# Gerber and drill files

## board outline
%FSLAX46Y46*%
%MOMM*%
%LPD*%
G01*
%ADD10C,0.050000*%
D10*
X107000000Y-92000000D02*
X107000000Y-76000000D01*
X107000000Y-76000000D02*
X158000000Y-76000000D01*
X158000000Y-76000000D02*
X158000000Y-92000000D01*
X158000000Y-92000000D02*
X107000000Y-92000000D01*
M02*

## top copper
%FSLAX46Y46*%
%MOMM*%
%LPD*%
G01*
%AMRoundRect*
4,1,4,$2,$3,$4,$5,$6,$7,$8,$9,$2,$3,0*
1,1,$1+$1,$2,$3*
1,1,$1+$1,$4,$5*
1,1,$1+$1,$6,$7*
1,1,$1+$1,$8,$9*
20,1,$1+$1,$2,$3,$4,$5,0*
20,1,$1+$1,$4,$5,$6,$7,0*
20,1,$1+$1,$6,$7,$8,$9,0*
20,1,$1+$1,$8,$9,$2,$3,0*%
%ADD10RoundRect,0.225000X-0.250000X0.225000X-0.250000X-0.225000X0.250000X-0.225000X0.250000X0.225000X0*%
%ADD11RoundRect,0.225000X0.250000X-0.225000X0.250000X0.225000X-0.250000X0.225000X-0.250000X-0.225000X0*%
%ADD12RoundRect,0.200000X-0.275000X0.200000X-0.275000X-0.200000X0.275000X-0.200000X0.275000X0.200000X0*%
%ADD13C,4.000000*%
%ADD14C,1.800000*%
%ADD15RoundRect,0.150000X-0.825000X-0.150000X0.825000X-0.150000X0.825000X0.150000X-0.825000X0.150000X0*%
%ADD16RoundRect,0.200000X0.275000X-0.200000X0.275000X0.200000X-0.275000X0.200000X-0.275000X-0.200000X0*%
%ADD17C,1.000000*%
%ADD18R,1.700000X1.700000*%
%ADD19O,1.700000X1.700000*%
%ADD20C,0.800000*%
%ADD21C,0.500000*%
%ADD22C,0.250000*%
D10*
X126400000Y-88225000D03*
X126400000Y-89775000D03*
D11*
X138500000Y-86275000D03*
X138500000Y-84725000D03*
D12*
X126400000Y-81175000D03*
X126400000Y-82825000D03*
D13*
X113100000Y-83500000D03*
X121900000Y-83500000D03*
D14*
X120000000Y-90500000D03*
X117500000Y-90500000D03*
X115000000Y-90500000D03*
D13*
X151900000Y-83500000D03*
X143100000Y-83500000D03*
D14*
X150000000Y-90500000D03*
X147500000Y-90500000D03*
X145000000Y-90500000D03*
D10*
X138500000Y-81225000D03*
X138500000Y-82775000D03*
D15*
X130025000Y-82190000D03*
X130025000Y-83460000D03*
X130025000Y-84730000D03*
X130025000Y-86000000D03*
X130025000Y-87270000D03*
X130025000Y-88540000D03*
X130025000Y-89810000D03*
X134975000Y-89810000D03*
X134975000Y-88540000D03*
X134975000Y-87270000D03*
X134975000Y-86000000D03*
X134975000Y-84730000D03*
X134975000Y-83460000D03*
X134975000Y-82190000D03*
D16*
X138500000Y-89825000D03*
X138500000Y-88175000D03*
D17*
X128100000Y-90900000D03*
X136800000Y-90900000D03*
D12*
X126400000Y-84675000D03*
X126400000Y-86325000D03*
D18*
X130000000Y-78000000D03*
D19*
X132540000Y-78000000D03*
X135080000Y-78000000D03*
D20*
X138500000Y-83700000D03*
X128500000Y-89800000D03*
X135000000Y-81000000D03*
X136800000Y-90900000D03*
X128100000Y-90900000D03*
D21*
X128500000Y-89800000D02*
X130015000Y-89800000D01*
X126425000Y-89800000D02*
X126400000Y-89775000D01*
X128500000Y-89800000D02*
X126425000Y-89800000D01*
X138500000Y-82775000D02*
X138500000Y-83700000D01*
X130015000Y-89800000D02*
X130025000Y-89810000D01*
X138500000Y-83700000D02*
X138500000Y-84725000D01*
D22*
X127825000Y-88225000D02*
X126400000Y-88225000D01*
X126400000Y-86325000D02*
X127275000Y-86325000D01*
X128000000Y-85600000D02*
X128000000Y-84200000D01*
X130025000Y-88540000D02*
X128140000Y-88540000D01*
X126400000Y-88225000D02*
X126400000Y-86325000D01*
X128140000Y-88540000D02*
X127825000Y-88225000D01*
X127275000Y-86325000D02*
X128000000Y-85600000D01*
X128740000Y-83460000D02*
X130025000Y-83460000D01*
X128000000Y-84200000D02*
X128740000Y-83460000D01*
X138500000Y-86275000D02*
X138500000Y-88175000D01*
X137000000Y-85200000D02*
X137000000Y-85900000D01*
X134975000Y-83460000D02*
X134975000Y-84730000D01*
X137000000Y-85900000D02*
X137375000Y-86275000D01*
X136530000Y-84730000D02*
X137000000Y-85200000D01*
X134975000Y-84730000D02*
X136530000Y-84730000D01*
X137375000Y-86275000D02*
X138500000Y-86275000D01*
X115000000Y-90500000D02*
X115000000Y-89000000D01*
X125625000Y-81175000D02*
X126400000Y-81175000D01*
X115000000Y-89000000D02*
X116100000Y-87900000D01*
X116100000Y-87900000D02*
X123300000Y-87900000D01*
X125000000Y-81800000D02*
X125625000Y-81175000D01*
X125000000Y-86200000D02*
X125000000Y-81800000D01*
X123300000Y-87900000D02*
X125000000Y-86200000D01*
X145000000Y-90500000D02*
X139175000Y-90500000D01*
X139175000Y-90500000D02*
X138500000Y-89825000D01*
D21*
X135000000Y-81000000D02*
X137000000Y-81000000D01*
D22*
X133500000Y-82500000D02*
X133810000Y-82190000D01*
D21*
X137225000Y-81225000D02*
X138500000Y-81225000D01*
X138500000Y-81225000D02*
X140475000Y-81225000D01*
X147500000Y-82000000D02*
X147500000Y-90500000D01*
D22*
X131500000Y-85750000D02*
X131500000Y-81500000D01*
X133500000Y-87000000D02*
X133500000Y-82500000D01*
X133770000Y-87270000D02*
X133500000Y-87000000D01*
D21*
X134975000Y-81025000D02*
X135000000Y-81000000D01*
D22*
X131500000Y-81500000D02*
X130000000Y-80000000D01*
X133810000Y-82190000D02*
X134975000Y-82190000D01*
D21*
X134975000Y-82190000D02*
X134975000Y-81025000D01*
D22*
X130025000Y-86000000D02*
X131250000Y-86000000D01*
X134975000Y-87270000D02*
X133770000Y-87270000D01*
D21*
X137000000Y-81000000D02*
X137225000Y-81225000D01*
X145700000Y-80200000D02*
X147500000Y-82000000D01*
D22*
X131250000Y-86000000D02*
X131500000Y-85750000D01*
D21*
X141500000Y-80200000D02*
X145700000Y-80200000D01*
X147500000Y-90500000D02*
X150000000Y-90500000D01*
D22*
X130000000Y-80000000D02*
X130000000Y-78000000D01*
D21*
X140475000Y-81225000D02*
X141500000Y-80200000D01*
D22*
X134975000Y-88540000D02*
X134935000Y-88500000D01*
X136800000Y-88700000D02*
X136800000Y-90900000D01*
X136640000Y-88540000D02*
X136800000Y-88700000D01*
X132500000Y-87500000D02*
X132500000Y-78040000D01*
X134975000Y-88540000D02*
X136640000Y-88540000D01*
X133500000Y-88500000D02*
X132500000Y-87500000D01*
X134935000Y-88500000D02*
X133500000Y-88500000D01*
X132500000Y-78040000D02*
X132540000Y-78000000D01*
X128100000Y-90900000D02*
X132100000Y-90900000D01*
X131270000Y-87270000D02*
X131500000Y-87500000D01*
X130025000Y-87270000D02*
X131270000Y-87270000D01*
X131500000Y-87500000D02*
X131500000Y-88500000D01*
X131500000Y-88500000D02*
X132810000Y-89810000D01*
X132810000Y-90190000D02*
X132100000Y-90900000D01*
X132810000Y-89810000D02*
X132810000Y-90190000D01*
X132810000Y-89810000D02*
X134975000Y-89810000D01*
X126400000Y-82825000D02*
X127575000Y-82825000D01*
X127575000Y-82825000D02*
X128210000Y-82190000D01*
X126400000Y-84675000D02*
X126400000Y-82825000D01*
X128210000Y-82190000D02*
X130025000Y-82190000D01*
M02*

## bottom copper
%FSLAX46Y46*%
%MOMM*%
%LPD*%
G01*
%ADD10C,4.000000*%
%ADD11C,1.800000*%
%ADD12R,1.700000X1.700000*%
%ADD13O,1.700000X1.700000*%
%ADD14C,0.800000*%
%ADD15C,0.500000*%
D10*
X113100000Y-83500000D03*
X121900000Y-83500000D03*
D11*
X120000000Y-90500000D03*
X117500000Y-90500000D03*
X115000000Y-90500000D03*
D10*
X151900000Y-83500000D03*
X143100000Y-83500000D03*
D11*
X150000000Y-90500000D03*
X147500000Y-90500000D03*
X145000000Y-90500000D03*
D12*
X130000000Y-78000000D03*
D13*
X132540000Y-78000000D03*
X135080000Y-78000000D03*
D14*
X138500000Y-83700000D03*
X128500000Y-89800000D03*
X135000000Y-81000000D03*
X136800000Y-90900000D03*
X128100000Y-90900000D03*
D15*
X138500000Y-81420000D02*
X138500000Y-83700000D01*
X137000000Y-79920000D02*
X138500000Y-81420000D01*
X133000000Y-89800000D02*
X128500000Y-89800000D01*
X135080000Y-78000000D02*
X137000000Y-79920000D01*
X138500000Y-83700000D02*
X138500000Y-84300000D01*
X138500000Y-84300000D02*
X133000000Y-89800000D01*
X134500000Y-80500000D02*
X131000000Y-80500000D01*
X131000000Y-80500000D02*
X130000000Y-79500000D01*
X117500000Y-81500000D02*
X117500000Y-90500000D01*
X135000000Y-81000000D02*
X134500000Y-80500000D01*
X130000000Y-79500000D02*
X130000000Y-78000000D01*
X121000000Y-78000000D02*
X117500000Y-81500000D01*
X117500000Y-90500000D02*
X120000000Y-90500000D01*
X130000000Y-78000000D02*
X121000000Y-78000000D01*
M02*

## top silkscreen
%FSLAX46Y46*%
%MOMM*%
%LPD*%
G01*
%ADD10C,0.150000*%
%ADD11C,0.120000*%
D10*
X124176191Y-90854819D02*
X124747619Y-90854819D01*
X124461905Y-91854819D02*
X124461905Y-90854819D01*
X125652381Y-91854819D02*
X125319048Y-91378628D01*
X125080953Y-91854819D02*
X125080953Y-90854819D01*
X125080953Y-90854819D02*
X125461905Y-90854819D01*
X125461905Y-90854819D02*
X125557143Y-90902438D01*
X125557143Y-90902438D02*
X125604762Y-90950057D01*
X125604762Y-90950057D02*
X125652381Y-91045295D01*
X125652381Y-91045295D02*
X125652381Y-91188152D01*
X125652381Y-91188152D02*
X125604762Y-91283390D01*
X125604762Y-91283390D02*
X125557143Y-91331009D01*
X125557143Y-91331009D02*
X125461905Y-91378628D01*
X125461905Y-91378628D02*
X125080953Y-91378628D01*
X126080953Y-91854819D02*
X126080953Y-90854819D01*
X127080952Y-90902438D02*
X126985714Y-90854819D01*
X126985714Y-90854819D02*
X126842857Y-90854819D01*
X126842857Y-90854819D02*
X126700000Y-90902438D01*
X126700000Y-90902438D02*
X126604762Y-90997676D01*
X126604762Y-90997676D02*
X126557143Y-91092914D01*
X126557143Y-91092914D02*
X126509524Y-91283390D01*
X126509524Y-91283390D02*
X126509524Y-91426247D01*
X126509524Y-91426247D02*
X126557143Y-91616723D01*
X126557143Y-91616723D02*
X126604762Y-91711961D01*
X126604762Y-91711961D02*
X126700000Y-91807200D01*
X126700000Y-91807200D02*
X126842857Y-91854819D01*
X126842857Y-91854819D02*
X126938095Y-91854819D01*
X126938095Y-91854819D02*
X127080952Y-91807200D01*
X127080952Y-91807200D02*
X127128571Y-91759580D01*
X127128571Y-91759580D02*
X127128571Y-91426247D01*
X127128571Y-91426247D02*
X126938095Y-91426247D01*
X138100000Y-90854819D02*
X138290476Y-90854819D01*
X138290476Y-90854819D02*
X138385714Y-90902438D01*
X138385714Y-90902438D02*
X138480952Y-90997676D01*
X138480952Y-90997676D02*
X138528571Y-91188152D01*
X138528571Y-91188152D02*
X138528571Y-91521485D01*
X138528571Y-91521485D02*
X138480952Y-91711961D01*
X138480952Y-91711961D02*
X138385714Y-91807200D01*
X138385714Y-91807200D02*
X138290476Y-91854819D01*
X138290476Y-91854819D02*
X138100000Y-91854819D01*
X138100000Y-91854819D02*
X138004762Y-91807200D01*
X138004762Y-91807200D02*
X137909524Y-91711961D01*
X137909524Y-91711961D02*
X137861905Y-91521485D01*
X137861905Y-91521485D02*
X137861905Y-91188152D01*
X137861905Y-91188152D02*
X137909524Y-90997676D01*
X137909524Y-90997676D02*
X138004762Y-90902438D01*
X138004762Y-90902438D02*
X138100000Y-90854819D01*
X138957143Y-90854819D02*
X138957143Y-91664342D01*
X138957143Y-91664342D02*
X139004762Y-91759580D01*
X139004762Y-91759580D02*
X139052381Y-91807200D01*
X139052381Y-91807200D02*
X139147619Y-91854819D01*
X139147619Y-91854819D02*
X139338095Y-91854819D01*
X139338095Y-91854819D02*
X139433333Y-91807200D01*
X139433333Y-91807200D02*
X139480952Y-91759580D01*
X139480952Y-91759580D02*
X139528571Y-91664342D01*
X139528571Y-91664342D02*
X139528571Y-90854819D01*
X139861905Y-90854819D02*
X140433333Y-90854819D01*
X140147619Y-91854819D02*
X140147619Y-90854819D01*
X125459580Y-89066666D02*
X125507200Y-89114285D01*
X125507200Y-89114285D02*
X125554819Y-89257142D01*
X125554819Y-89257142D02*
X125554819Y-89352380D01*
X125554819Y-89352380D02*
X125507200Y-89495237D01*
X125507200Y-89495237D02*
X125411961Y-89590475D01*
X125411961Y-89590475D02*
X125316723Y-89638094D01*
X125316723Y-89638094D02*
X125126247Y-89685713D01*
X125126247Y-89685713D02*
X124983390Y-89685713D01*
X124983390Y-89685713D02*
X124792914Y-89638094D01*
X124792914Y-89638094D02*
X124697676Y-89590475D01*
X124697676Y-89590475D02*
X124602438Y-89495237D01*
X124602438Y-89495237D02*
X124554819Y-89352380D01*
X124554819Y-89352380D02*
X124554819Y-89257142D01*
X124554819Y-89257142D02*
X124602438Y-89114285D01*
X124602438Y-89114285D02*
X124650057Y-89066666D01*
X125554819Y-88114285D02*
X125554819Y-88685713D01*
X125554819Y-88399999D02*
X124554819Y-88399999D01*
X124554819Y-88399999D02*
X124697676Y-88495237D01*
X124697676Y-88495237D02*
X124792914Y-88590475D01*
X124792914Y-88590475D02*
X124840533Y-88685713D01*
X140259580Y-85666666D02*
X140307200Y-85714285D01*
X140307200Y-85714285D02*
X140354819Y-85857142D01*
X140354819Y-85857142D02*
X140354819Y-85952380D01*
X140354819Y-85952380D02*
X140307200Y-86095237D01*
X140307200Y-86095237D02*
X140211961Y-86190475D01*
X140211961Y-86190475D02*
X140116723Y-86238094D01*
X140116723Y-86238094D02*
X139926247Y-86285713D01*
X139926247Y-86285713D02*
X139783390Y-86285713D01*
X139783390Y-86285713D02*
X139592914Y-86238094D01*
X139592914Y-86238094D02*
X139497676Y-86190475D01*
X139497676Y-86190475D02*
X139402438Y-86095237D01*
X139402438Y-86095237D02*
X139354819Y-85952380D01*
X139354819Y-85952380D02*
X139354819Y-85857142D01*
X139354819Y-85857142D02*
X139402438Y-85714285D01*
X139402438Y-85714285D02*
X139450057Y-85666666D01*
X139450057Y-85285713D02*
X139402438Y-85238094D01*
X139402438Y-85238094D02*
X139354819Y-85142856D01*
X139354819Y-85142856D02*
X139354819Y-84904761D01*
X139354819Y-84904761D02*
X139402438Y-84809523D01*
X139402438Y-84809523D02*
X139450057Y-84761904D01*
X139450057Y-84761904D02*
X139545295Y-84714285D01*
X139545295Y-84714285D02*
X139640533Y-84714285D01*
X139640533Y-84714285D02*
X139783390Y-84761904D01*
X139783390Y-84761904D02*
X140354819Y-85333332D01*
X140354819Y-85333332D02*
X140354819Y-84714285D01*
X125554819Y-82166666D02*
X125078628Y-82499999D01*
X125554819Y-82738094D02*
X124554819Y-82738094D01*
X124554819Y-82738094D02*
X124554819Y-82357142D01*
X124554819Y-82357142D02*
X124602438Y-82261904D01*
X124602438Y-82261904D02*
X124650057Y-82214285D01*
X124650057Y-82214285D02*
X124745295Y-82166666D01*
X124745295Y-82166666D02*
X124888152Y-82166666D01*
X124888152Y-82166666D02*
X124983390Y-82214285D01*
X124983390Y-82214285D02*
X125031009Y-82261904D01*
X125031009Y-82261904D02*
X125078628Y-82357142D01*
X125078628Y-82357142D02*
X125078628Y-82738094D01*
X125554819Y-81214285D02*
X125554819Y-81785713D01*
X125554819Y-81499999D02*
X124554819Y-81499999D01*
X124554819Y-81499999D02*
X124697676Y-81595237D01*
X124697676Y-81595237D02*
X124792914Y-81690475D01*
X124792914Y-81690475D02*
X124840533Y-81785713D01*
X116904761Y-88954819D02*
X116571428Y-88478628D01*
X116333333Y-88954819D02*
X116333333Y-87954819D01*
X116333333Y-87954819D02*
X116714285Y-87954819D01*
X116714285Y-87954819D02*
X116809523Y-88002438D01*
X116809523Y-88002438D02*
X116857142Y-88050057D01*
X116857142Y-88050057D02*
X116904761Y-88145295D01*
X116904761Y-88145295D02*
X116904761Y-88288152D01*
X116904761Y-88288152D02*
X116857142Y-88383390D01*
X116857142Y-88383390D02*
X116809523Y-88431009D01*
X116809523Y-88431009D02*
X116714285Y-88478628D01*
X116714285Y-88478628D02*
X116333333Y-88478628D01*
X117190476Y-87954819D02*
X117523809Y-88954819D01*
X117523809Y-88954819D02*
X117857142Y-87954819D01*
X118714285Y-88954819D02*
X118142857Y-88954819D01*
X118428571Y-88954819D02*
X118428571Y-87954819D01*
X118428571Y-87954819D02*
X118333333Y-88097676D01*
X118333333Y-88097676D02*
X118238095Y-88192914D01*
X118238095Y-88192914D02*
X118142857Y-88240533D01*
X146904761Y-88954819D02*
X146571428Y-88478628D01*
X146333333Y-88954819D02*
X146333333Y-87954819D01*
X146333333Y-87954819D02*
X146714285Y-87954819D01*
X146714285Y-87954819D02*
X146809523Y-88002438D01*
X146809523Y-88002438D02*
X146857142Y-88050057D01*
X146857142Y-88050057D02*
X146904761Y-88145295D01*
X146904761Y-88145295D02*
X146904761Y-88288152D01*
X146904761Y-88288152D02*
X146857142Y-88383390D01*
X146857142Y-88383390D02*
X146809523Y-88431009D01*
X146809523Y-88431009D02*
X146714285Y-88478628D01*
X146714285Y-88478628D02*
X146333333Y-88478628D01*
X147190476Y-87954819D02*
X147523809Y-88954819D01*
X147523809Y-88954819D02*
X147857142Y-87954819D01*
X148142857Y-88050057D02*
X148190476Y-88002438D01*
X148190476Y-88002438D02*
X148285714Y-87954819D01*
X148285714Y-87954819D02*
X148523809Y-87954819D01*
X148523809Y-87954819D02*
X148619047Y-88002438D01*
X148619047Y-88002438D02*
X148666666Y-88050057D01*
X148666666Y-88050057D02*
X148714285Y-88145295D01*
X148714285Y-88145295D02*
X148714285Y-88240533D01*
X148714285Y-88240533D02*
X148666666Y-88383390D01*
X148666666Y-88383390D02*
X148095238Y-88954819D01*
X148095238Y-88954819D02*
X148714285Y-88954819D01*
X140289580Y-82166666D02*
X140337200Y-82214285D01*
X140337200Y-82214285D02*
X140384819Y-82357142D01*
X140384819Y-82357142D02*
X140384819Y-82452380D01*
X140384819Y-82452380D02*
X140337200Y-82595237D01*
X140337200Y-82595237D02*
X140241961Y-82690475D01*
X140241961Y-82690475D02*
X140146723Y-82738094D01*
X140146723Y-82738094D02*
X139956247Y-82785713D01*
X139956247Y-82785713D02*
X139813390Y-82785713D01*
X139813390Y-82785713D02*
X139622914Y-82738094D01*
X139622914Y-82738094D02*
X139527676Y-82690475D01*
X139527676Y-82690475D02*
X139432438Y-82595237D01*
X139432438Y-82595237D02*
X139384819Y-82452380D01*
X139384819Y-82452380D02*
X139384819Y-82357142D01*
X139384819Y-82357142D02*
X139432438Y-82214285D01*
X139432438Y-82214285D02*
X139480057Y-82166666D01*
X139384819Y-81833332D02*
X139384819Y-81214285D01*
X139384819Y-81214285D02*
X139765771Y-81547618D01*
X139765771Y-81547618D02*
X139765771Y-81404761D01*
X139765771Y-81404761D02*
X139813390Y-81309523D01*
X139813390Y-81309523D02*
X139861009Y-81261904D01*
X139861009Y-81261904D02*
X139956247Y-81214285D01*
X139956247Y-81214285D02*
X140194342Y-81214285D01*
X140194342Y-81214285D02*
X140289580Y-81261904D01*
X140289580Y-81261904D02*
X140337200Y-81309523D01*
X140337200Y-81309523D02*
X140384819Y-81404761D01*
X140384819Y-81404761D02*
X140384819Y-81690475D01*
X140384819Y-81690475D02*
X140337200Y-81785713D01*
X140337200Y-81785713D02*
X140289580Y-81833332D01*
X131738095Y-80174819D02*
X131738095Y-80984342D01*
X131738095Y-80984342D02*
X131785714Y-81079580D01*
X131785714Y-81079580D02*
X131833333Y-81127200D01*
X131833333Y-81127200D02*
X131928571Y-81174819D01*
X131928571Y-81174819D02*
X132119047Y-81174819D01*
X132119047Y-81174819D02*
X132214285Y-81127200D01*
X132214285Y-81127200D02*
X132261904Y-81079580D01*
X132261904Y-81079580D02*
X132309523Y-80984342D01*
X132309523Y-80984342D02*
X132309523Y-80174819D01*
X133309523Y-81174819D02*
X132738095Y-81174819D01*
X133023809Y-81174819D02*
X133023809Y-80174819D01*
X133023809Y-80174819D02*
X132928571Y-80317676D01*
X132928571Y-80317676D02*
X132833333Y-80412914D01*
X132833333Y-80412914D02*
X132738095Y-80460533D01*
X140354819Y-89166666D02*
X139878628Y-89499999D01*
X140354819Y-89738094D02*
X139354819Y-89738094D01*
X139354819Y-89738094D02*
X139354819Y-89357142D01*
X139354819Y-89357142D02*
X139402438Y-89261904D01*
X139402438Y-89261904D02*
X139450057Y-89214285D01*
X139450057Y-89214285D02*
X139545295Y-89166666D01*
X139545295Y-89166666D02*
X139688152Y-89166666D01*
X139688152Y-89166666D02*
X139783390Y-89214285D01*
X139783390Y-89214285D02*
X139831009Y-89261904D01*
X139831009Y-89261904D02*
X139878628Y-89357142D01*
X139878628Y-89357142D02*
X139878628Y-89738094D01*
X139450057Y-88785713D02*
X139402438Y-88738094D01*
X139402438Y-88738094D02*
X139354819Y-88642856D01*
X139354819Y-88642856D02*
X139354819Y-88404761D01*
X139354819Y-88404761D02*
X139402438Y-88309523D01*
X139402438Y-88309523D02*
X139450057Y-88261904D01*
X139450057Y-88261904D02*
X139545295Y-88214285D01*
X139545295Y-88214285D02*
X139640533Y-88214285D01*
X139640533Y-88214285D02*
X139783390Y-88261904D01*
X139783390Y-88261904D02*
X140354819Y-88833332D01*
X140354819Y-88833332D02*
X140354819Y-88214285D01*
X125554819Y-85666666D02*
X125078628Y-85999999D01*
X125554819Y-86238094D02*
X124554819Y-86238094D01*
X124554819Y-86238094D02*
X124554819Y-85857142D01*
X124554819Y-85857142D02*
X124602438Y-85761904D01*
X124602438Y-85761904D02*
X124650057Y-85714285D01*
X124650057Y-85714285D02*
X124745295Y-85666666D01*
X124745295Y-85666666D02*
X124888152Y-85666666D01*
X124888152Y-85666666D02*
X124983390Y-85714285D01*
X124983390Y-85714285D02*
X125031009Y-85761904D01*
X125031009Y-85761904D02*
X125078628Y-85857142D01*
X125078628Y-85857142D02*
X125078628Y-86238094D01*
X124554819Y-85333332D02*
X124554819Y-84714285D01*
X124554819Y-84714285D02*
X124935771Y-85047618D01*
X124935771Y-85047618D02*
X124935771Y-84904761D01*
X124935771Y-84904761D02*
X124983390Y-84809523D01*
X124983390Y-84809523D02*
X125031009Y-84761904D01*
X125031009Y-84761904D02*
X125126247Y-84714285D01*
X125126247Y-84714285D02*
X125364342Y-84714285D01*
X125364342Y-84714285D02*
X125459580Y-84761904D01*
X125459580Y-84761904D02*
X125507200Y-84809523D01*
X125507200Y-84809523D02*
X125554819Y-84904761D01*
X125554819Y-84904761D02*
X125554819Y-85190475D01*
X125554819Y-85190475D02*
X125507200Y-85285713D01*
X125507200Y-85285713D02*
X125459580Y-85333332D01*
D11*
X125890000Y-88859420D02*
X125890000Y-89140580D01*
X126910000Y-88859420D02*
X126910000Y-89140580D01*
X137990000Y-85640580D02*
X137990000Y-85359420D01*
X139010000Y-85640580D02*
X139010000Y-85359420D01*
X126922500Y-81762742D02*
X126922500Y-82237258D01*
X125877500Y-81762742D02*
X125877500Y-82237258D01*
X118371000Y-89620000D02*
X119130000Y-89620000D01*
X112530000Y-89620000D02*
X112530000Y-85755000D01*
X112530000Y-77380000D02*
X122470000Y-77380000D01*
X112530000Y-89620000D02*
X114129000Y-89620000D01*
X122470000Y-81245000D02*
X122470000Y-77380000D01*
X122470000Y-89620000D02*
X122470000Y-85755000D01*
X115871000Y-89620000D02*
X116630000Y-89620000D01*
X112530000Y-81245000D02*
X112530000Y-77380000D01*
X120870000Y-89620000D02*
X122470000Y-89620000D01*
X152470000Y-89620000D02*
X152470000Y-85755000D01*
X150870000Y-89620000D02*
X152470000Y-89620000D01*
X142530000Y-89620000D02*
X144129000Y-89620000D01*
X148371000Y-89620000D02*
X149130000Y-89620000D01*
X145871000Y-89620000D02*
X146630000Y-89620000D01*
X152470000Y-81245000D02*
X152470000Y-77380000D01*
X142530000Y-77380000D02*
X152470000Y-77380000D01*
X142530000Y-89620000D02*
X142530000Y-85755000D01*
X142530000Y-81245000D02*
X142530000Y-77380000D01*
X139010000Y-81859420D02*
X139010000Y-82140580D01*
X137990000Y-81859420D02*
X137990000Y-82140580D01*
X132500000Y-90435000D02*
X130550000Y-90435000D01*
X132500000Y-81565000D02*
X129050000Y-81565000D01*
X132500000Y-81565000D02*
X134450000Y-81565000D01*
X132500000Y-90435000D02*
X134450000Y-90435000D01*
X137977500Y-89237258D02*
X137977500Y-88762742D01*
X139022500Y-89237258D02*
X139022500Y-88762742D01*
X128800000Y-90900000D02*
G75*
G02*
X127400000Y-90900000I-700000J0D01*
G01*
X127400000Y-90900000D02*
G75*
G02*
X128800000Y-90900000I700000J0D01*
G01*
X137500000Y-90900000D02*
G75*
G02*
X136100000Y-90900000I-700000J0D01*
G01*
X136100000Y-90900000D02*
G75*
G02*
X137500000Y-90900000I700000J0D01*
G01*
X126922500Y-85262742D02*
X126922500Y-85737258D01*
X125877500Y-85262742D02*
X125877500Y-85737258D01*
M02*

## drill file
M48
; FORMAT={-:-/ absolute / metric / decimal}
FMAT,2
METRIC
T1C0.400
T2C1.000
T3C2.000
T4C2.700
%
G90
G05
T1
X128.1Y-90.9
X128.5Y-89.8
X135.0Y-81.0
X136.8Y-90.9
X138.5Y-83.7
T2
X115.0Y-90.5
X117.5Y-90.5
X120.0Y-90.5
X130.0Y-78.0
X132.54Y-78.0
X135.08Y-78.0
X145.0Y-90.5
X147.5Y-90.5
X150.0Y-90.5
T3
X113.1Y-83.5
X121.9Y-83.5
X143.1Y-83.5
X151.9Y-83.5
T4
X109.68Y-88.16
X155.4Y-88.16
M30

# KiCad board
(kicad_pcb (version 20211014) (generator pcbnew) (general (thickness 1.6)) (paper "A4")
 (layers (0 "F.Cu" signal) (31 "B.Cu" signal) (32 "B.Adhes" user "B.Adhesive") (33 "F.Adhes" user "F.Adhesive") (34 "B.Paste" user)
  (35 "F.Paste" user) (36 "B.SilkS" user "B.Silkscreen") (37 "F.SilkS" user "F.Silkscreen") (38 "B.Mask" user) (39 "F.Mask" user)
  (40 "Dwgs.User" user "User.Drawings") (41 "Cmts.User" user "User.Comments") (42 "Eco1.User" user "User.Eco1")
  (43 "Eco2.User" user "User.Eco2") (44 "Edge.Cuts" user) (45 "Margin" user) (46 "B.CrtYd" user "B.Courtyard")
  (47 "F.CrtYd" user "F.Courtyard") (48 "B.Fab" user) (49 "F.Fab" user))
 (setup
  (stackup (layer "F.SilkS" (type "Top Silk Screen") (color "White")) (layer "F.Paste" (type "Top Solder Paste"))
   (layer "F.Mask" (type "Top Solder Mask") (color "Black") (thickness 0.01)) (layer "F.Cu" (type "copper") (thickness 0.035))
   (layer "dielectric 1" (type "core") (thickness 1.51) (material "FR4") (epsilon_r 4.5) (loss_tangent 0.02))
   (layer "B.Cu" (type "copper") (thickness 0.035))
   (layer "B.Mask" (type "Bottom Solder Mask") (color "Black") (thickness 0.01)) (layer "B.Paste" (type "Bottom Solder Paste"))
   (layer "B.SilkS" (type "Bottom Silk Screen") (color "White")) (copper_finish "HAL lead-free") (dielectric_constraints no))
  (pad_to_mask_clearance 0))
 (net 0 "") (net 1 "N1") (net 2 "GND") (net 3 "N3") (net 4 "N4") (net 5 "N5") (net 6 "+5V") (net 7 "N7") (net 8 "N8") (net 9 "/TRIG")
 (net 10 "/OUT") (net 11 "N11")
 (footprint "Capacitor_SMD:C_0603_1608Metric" (layer "F.Cu") (at 126.4 89 -90)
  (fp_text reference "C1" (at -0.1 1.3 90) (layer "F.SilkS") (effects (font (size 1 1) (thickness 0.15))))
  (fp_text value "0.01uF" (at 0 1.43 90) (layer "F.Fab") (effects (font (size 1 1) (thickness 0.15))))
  (fp_line (start -0.14058 0.51) (end 0.14058 0.51) (layer "F.SilkS") (width 0.12))
  (fp_line (start -0.14058 -0.51) (end 0.14058 -0.51) (layer "F.SilkS") (width 0.12))
  (pad "1" smd roundrect locked (at -0.775 0 270) (size 0.9 0.95) (layers "F.Cu" "F.Paste" "F.Mask") (roundrect_rratio 0.25) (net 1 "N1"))
  (pad "2" smd roundrect locked (at 0.775 0 270) (size 0.9 0.95) (layers "F.Cu" "F.Paste" "F.Mask") (roundrect_rratio 0.25) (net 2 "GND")))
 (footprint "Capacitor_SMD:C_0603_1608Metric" (layer "F.Cu") (at 138.5 85.5 90)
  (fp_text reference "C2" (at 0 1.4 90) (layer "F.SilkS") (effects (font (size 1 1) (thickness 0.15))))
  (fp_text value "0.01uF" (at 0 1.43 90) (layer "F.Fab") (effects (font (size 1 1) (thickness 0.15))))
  (fp_line (start -0.14058 -0.51) (end 0.14058 -0.51) (layer "F.SilkS") (width 0.12))
  (fp_line (start -0.14058 0.51) (end 0.14058 0.51) (layer "F.SilkS") (width 0.12))
  (pad "1" smd roundrect locked (at -0.775 0 90) (size 0.9 0.95) (layers "F.Cu" "F.Paste" "F.Mask") (roundrect_rratio 0.25) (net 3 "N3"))
  (pad "2" smd roundrect locked (at 0.775 0 90) (size 0.9 0.95) (layers "F.Cu" "F.Paste" "F.Mask") (roundrect_rratio 0.25) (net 2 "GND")))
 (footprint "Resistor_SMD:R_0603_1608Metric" (layer "F.Cu") (at 126.4 82 -90)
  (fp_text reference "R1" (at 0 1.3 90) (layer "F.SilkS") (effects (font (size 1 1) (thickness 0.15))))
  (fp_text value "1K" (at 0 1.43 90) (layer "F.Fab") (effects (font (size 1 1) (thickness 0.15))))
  (fp_line (start -0.237258 -0.5225) (end 0.237258 -0.5225) (layer "F.SilkS") (width 0.12))
  (fp_line (start -0.237258 0.5225) (end 0.237258 0.5225) (layer "F.SilkS") (width 0.12))
  (pad "1" smd roundrect locked (at -0.825 0 270) (size 0.8 0.95) (layers "F.Cu" "F.Paste" "F.Mask") (roundrect_rratio 0.25) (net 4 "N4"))
  (pad "2" smd roundrect locked (at 0.825 0 270) (size 0.8 0.95) (layers "F.Cu" "F.Paste" "F.Mask") (roundrect_rratio 0.25) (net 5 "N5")))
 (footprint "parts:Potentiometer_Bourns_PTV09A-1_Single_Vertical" (layer "F.Cu") (at 120 90.5 90)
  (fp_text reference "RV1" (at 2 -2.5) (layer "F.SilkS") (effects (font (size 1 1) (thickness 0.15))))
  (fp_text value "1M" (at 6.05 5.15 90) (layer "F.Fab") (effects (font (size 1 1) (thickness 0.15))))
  (fp_line (start 0.88 -1.629) (end 0.88 -0.87) (layer "F.SilkS") (width 0.12))
  (fp_line (start 0.88 -7.47) (end 4.745 -7.47) (layer "F.SilkS") (width 0.12))
  (fp_line (start 13.12 -7.47) (end 13.12 2.47) (layer "F.SilkS") (width 0.12))
  (fp_line (start 0.88 -7.47) (end 0.88 -5.871) (layer "F.SilkS") (width 0.12))
  (fp_line (start 9.255 2.47) (end 13.12 2.47) (layer "F.SilkS") (width 0.12))
  (fp_line (start 0.88 2.47) (end 4.745 2.47) (layer "F.SilkS") (width 0.12))
  (fp_line (start 0.88 -4.129) (end 0.88 -3.37) (layer "F.SilkS") (width 0.12))
  (fp_line (start 9.255 -7.47) (end 13.12 -7.47) (layer "F.SilkS") (width 0.12))
  (fp_line (start 0.88 0.87) (end 0.88 2.47) (layer "F.SilkS") (width 0.12))
  (pad "" np_thru_hole circle locked (at 7 -6.9 90) (size 4 4) (drill 2) (layers *.Cu *.Mask))
  (pad "" np_thru_hole circle locked (at 7 1.9 90) (size 4 4) (drill 2) (layers *.Cu *.Mask))
  (pad "1" thru_hole circle locked (at 0 0 90) (size 1.8 1.8) (drill 1) (layers *.Cu *.Mask) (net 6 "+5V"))
  (pad "2" thru_hole circle locked (at 0 -2.5 90) (size 1.8 1.8) (drill 1) (layers *.Cu *.Mask) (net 6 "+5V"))
  (pad "3" thru_hole circle locked (at 0 -5 90) (size 1.8 1.8) (drill 1) (layers *.Cu *.Mask) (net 4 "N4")))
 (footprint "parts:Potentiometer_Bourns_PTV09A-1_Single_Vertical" (layer "F.Cu") (at 150 90.5 90)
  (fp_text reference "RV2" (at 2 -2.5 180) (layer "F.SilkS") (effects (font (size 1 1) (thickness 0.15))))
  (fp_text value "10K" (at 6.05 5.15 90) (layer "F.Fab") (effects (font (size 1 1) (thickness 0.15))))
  (fp_line (start 0.88 2.47) (end 4.745 2.47) (layer "F.SilkS") (width 0.12))
  (fp_line (start 0.88 0.87) (end 0.88 2.47) (layer "F.SilkS") (width 0.12))
  (fp_line (start 0.88 -7.47) (end 0.88 -5.871) (layer "F.SilkS") (width 0.12))
  (fp_line (start 0.88 -1.629) (end 0.88 -0.87) (layer "F.SilkS") (width 0.12))
  (fp_line (start 0.88 -4.129) (end 0.88 -3.37) (layer "F.SilkS") (width 0.12))
  (fp_line (start 9.255 2.47) (end 13.12 2.47) (layer "F.SilkS") (width 0.12))
  (fp_line (start 13.12 -7.47) (end 13.12 2.47) (layer "F.SilkS") (width 0.12))
  (fp_line (start 0.88 -7.47) (end 4.745 -7.47) (layer "F.SilkS") (width 0.12))
  (fp_line (start 9.255 -7.47) (end 13.12 -7.47) (layer "F.SilkS") (width 0.12))
  (pad "" np_thru_hole circle locked (at 7 1.9 90) (size 4 4) (drill 2) (layers *.Cu *.Mask))
  (pad "" np_thru_hole circle locked (at 7 -6.9 90) (size 4 4) (drill 2) (layers *.Cu *.Mask))
  (pad "1" thru_hole circle locked (at 0 0 90) (size 1.8 1.8) (drill 1) (layers *.Cu *.Mask) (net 6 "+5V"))
  (pad "2" thru_hole circle locked (at 0 -2.5 90) (size 1.8 1.8) (drill 1) (layers *.Cu *.Mask) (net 6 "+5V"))
  (pad "3" thru_hole circle locked (at 0 -5 90) (size 1.8 1.8) (drill 1) (layers *.Cu *.Mask) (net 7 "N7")))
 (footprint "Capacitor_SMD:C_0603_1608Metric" (layer "F.Cu") (at 138.5 82 -90)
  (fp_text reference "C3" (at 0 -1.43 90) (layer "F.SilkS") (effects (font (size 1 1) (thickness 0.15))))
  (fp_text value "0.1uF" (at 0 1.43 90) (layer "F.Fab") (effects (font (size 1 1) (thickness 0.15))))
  (fp_line (start -0.14058 -0.51) (end 0.14058 -0.51) (layer "F.SilkS") (width 0.12))
  (fp_line (start -0.14058 0.51) (end 0.14058 0.51) (layer "F.SilkS") (width 0.12))
  (pad "1" smd roundrect locked (at -0.775 0 270) (size 0.9 0.95) (layers "F.Cu" "F.Paste" "F.Mask") (roundrect_rratio 0.25) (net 6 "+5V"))
  (pad "2" smd roundrect locked (at 0.775 0 270) (size 0.9 0.95) (layers "F.Cu" "F.Paste" "F.Mask") (roundrect_rratio 0.25) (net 2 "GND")))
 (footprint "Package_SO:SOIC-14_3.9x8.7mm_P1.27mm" (layer "F.Cu") (at 132.5 86)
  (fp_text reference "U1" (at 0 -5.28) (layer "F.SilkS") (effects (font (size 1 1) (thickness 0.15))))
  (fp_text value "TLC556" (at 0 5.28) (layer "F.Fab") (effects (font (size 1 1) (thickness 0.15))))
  (fp_line (start 0 4.435) (end -1.95 4.435) (layer "F.SilkS") (width 0.12))
  (fp_line (start 0 -4.435) (end -3.45 -4.435) (layer "F.SilkS") (width 0.12))
  (fp_line (start 0 -4.435) (end 1.95 -4.435) (layer "F.SilkS") (width 0.12))
  (fp_line (start 0 4.435) (end 1.95 4.435) (layer "F.SilkS") (width 0.12))
  (pad "1" smd roundrect locked (at -2.475 -3.81) (size 1.95 0.6) (layers "F.Cu" "F.Paste" "F.Mask") (roundrect_rratio 0.25) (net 5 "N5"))
  (pad "2" smd roundrect locked (at -2.475 -2.54) (size 1.95 0.6) (layers "F.Cu" "F.Paste" "F.Mask") (roundrect_rratio 0.25) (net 1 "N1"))
  (pad "3" smd roundrect locked (at -2.475 -1.27) (size 1.95 0.6) (layers "F.Cu" "F.Paste" "F.Mask") (roundrect_rratio 0.25) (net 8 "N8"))
  (pad "4" smd roundrect locked (at -2.475 0) (size 1.95 0.6) (layers "F.Cu" "F.Paste" "F.Mask") (roundrect_rratio 0.25) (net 6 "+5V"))
  (pad "5" smd roundrect locked (at -2.475 1.27) (size 1.95 0.6) (layers "F.Cu" "F.Paste" "F.Mask") (roundrect_rratio 0.25) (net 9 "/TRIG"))
  (pad "6" smd roundrect locked (at -2.475 2.54) (size 1.95 0.6) (layers "F.Cu" "F.Paste" "F.Mask") (roundrect_rratio 0.25) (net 1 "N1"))
  (pad "7" smd roundrect locked (at -2.475 3.81) (size 1.95 0.6) (layers "F.Cu" "F.Paste" "F.Mask") (roundrect_rratio 0.25) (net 2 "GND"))
  (pad "8" smd roundrect locked (at 2.475 3.81) (size 1.95 0.6) (layers "F.Cu" "F.Paste" "F.Mask") (roundrect_rratio 0.25) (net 9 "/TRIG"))
  (pad "9" smd roundrect locked (at 2.475 2.54) (size 1.95 0.6) (layers "F.Cu" "F.Paste" "F.Mask") (roundrect_rratio 0.25) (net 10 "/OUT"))
  (pad "10" smd roundrect locked (at 2.475 1.27) (size 1.95 0.6) (layers "F.Cu" "F.Paste" "F.Mask") (roundrect_rratio 0.25) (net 6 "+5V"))
  (pad "11" smd roundrect locked (at 2.475 0) (size 1.95 0.6) (layers "F.Cu" "F.Paste" "F.Mask") (roundrect_rratio 0.25) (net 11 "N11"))
  (pad "12" smd roundrect locked (at 2.475 -1.27) (size 1.95 0.6) (layers "F.Cu" "F.Paste" "F.Mask") (roundrect_rratio 0.25) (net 3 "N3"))
  (pad "13" smd roundrect locked (at 2.475 -2.54) (size 1.95 0.6) (layers "F.Cu" "F.Paste" "F.Mask") (roundrect_rratio 0.25) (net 3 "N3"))
  (pad "14" smd roundrect locked (at 2.475 -3.81) (size 1.95 0.6) (layers "F.Cu" "F.Paste" "F.Mask") (roundrect_rratio 0.25) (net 6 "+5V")))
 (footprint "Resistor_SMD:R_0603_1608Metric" (layer "F.Cu") (at 138.5 89 90)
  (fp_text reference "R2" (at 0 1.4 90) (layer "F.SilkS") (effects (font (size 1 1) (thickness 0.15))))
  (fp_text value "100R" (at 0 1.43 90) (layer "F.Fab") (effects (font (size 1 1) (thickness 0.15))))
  (fp_line (start -0.237258 -0.5225) (end 0.237258 -0.5225) (layer "F.SilkS") (width 0.12))
  (fp_line (start -0.237258 0.5225) (end 0.237258 0.5225) (layer "F.SilkS") (width 0.12))
  (pad "1" smd roundrect locked (at -0.825 0 90) (size 0.8 0.95) (layers "F.Cu" "F.Paste" "F.Mask") (roundrect_rratio 0.25) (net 7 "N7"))
  (pad "2" smd roundrect locked (at 0.825 0 90) (size 0.8 0.95) (layers "F.Cu" "F.Paste" "F.Mask") (roundrect_rratio 0.25) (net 3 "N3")))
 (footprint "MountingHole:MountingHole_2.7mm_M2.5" (layer "F.Cu") (at 109.68 88.16)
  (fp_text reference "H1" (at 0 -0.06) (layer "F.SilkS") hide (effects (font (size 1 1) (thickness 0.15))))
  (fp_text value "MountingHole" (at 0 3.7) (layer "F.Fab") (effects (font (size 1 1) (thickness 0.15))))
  (pad "" np_thru_hole circle locked (at 0 0) (size 2.7 2.7) (drill 2.7) (layers *.Cu *.Mask)))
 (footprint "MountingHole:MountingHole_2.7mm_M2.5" (layer "F.Cu") (at 155.4 88.16)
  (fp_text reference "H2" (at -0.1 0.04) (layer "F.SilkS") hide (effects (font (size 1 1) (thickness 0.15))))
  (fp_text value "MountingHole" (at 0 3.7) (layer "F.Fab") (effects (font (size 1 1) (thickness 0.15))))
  (pad "" np_thru_hole circle locked (at 0 0) (size 2.7 2.7) (drill 2.7) (layers *.Cu *.Mask)))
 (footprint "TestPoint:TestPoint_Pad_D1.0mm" (layer "F.Cu") (at 128.1 90.9)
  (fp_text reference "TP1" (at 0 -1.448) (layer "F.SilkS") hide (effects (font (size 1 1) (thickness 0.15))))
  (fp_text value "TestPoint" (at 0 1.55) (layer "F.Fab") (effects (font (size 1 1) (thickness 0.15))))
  (fp_circle (center 0 0) (end 0 0.7) (layer "F.SilkS") (width 0.12) (fill none))
  (pad "1" smd circle locked (at 0 0) (size 1 1) (layers "F.Cu" "F.Mask") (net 9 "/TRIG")))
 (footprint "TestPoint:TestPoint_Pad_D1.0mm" (layer "F.Cu") (at 136.8 90.9)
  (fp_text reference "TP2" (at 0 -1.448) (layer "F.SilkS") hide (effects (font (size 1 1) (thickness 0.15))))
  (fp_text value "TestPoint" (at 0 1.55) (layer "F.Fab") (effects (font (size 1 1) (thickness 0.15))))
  (fp_circle (center 0 0) (end 0 0.7) (layer "F.SilkS") (width 0.12) (fill none))
  (pad "1" smd circle locked (at 0 0) (size 1 1) (layers "F.Cu" "F.Mask") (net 10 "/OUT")))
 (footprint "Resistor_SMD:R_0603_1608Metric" (layer "F.Cu") (at 126.4 85.5 -90)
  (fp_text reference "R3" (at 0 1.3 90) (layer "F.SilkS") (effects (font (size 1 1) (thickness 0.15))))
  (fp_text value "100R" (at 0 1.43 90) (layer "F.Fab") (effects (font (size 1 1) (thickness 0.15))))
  (fp_line (start -0.237258 -0.5225) (end 0.237258 -0.5225) (layer "F.SilkS") (width 0.12))
  (fp_line (start -0.237258 0.5225) (end 0.237258 0.5225) (layer "F.SilkS") (width 0.12))
  (pad "1" smd roundrect locked (at -0.825 0 270) (size 0.8 0.95) (layers "F.Cu" "F.Paste" "F.Mask") (roundrect_rratio 0.25) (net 5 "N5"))
  (pad "2" smd roundrect locked (at 0.825 0 270) (size 0.8 0.95) (layers "F.Cu" "F.Paste" "F.Mask") (roundrect_rratio 0.25) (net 1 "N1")))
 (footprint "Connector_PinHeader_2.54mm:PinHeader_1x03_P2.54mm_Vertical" (layer "B.Cu") (at 130 78 -90)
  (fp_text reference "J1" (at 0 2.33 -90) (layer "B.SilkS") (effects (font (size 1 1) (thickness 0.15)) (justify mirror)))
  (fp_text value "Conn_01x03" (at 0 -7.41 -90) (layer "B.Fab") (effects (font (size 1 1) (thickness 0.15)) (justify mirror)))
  (pad "1" thru_hole rect locked (at 0 0 270) (size 1.7 1.7) (drill 1) (layers *.Cu *.Mask) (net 6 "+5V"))
  (pad "2" thru_hole oval locked (at 0 -2.54 270) (size 1.7 1.7) (drill 1) (layers *.Cu *.Mask) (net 10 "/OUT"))
  (pad "3" thru_hole oval locked (at 0 -5.08 270) (size 1.7 1.7) (drill 1) (layers *.Cu *.Mask) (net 2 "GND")))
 (gr_line (start 107 92) (end 107 76) (layer "Edge.Cuts") (width 0.05))
 (gr_line (start 107 76) (end 158 76) (layer "Edge.Cuts") (width 0.05))
 (gr_line (start 158 76) (end 158 92) (layer "Edge.Cuts") (width 0.05))
 (gr_line (start 158 92) (end 107 92) (layer "Edge.Cuts") (width 0.05))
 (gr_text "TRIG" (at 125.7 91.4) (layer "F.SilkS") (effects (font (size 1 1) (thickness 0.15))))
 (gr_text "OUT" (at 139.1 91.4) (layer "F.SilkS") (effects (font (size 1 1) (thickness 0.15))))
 (segment (start 128.5 89.8) (end 130.015 89.8) (width 0.5) (layer "F.Cu") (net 2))
 (segment (start 126.425 89.8) (end 126.4 89.775) (width 0.5) (layer "F.Cu") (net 2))
 (segment (start 128.5 89.8) (end 126.425 89.8) (width 0.5) (layer "F.Cu") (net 2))
 (segment (start 138.5 82.775) (end 138.5 83.7) (width 0.5) (layer "F.Cu") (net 2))
 (segment (start 130.015 89.8) (end 130.025 89.81) (width 0.5) (layer "F.Cu") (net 2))
 (segment (start 138.5 83.7) (end 138.5 84.725) (width 0.5) (layer "F.Cu") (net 2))
 (via (at 138.5 83.7) (size 0.8) (drill 0.4) (layers "F.Cu" "B.Cu") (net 2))
 (via (at 128.5 89.8) (size 0.8) (drill 0.4) (layers "F.Cu" "B.Cu") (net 2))
 (segment (start 138.5 81.42) (end 138.5 83.7) (width 0.5) (layer "B.Cu") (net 2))
 (segment (start 137 79.92) (end 138.5 81.42) (width 0.5) (layer "B.Cu") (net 2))
 (segment (start 133 89.8) (end 128.5 89.8) (width 0.5) (layer "B.Cu") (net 2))
 (segment (start 135.08 78) (end 137 79.92) (width 0.5) (layer "B.Cu") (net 2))
 (segment (start 138.5 83.7) (end 138.5 84.3) (width 0.5) (layer "B.Cu") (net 2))
 (segment (start 138.5 84.3) (end 133 89.8) (width 0.5) (layer "B.Cu") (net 2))
 (segment (start 127.825 88.225) (end 126.4 88.225) (width 0.25) (layer "F.Cu") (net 1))
 (segment (start 126.4 86.325) (end 127.275 86.325) (width 0.25) (layer "F.Cu") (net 1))
 (segment (start 128 85.6) (end 128 84.2) (width 0.25) (layer "F.Cu") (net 1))
 (segment (start 130.025 88.54) (end 128.14 88.54) (width 0.25) (layer "F.Cu") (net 1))
 (segment (start 126.4 88.225) (end 126.4 86.325) (width 0.25) (layer "F.Cu") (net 1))
 (segment (start 128.14 88.54) (end 127.825 88.225) (width 0.25) (layer "F.Cu") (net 1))
 (segment (start 127.275 86.325) (end 128 85.6) (width 0.25) (layer "F.Cu") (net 1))
 (segment (start 128.74 83.46) (end 130.025 83.46) (width 0.25) (layer "F.Cu") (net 1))
 (segment (start 128 84.2) (end 128.74 83.46) (width 0.25) (layer "F.Cu") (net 1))
 (segment (start 138.5 86.275) (end 138.5 88.175) (width 0.25) (layer "F.Cu") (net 3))
 (segment (start 137 85.2) (end 137 85.9) (width 0.25) (layer "F.Cu") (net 3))
 (segment (start 134.975 83.46) (end 134.975 84.73) (width 0.25) (layer "F.Cu") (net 3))
 (segment (start 137 85.9) (end 137.375 86.275) (width 0.25) (layer "F.Cu") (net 3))
 (segment (start 136.53 84.73) (end 137 85.2) (width 0.25) (layer "F.Cu") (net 3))
 (segment (start 134.975 84.73) (end 136.53 84.73) (width 0.25) (layer "F.Cu") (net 3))
 (segment (start 137.375 86.275) (end 138.5 86.275) (width 0.25) (layer "F.Cu") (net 3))
 (segment (start 115 90.5) (end 115 89) (width 0.25) (layer "F.Cu") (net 4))
 (segment (start 125.625 81.175) (end 126.4 81.175) (width 0.25) (layer "F.Cu") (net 4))
 (segment (start 115 89) (end 116.1 87.9) (width 0.25) (layer "F.Cu") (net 4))
 (segment (start 116.1 87.9) (end 123.3 87.9) (width 0.25) (layer "F.Cu") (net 4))
 (segment (start 125 81.8) (end 125.625 81.175) (width 0.25) (layer "F.Cu") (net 4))
 (segment (start 125 86.2) (end 125 81.8) (width 0.25) (layer "F.Cu") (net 4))
 (segment (start 123.3 87.9) (end 125 86.2) (width 0.25) (layer "F.Cu") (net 4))
 (segment (start 145 90.5) (end 139.175 90.5) (width 0.25) (layer "F.Cu") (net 7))
 (segment (start 139.175 90.5) (end 138.5 89.825) (width 0.25) (layer "F.Cu") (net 7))
 (segment (start 135 81) (end 137 81) (width 0.5) (layer "F.Cu") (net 6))
 (segment (start 133.5 82.5) (end 133.81 82.19) (width 0.25) (layer "F.Cu") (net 6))
 (segment (start 137.225 81.225) (end 138.5 81.225) (width 0.5) (layer "F.Cu") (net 6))
 (segment (start 138.5 81.225) (end 140.475 81.225) (width 0.5) (layer "F.Cu") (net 6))
 (segment (start 147.5 82) (end 147.5 90.5) (width 0.5) (layer "F.Cu") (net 6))
 (segment (start 131.5 85.75) (end 131.5 81.5) (width 0.25) (layer "F.Cu") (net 6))
 (segment (start 133.5 87) (end 133.5 82.5) (width 0.25) (layer "F.Cu") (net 6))
 (segment (start 133.77 87.27) (end 133.5 87) (width 0.25) (layer "F.Cu") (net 6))
 (segment (start 134.975 81.025) (end 135 81) (width 0.5) (layer "F.Cu") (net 6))
 (segment (start 131.5 81.5) (end 130 80) (width 0.25) (layer "F.Cu") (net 6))
 (segment (start 133.81 82.19) (end 134.975 82.19) (width 0.25) (layer "F.Cu") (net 6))
 (segment (start 134.975 82.19) (end 134.975 81.025) (width 0.5) (layer "F.Cu") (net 6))
 (segment (start 130.025 86) (end 131.25 86) (width 0.25) (layer "F.Cu") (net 6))
 (segment (start 134.975 87.27) (end 133.77 87.27) (width 0.25) (layer "F.Cu") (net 6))
 (segment (start 137 81) (end 137.225 81.225) (width 0.5) (layer "F.Cu") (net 6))
 (segment (start 145.7 80.2) (end 147.5 82) (width 0.5) (layer "F.Cu") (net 6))
 (segment (start 131.25 86) (end 131.5 85.75) (width 0.25) (layer "F.Cu") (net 6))
 (segment (start 141.5 80.2) (end 145.7 80.2) (width 0.5) (layer "F.Cu") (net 6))
 (segment (start 147.5 90.5) (end 150 90.5) (width 0.5) (layer "F.Cu") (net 6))
 (segment (start 130 80) (end 130 78) (width 0.25) (layer "F.Cu") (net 6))
 (segment (start 140.475 81.225) (end 141.5 80.2) (width 0.5) (layer "F.Cu") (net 6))
 (via (at 135 81) (size 0.8) (drill 0.4) (layers "F.Cu" "B.Cu") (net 6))
 (segment (start 134.5 80.5) (end 131 80.5) (width 0.5) (layer "B.Cu") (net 6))
 (segment (start 131 80.5) (end 130 79.5) (width 0.5) (layer "B.Cu") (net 6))
 (segment (start 117.5 81.5) (end 117.5 90.5) (width 0.5) (layer "B.Cu") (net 6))
 (segment (start 135 81) (end 134.5 80.5) (width 0.5) (layer "B.Cu") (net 6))
 (segment (start 130 79.5) (end 130 78) (width 0.5) (layer "B.Cu") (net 6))
 (segment (start 121 78) (end 117.5 81.5) (width 0.5) (layer "B.Cu") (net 6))
 (segment (start 117.5 90.5) (end 120 90.5) (width 0.5) (layer "B.Cu") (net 6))
 (segment (start 130 78) (end 121 78) (width 0.5) (layer "B.Cu") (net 6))
 (segment (start 134.975 88.54) (end 134.935 88.5) (width 0.25) (layer "F.Cu") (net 10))
 (segment (start 136.8 88.7) (end 136.8 90.9) (width 0.25) (layer "F.Cu") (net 10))
 (segment (start 136.64 88.54) (end 136.8 88.7) (width 0.25) (layer "F.Cu") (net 10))
 (segment (start 132.5 87.5) (end 132.5 78.04) (width 0.25) (layer "F.Cu") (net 10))
 (segment (start 134.975 88.54) (end 136.64 88.54) (width 0.25) (layer "F.Cu") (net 10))
 (segment (start 133.5 88.5) (end 132.5 87.5) (width 0.25) (layer "F.Cu") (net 10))
 (segment (start 134.935 88.5) (end 133.5 88.5) (width 0.25) (layer "F.Cu") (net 10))
 (segment (start 132.5 78.04) (end 132.54 78) (width 0.25) (layer "F.Cu") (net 10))
 (via (at 136.8 90.9) (size 0.8) (drill 0.4) (layers "F.Cu" "B.Cu") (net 10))
 (segment (start 128.1 90.9) (end 132.1 90.9) (width 0.25) (layer "F.Cu") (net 9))
 (segment (start 131.27 87.27) (end 131.5 87.5) (width 0.25) (layer "F.Cu") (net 9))
 (segment (start 130.025 87.27) (end 131.27 87.27) (width 0.25) (layer "F.Cu") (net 9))
 (segment (start 131.5 87.5) (end 131.5 88.5) (width 0.25) (layer "F.Cu") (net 9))
 (segment (start 131.5 88.5) (end 132.81 89.81) (width 0.25) (layer "F.Cu") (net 9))
 (segment (start 132.81 90.19) (end 132.1 90.9) (width 0.25) (layer "F.Cu") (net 9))
 (segment (start 132.81 89.81) (end 132.81 90.19) (width 0.25) (layer "F.Cu") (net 9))
 (segment (start 132.81 89.81) (end 134.975 89.81) (width 0.25) (layer "F.Cu") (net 9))
 (via (at 128.1 90.9) (size 0.8) (drill 0.4) (layers "F.Cu" "B.Cu") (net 9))
 (segment (start 126.4 82.825) (end 127.575 82.825) (width 0.25) (layer "F.Cu") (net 5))
 (segment (start 127.575 82.825) (end 128.21 82.19) (width 0.25) (layer "F.Cu") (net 5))
 (segment (start 126.4 84.675) (end 126.4 82.825) (width 0.25) (layer "F.Cu") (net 5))
 (segment (start 128.21 82.19) (end 130.025 82.19) (width 0.25) (layer "F.Cu") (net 5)))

